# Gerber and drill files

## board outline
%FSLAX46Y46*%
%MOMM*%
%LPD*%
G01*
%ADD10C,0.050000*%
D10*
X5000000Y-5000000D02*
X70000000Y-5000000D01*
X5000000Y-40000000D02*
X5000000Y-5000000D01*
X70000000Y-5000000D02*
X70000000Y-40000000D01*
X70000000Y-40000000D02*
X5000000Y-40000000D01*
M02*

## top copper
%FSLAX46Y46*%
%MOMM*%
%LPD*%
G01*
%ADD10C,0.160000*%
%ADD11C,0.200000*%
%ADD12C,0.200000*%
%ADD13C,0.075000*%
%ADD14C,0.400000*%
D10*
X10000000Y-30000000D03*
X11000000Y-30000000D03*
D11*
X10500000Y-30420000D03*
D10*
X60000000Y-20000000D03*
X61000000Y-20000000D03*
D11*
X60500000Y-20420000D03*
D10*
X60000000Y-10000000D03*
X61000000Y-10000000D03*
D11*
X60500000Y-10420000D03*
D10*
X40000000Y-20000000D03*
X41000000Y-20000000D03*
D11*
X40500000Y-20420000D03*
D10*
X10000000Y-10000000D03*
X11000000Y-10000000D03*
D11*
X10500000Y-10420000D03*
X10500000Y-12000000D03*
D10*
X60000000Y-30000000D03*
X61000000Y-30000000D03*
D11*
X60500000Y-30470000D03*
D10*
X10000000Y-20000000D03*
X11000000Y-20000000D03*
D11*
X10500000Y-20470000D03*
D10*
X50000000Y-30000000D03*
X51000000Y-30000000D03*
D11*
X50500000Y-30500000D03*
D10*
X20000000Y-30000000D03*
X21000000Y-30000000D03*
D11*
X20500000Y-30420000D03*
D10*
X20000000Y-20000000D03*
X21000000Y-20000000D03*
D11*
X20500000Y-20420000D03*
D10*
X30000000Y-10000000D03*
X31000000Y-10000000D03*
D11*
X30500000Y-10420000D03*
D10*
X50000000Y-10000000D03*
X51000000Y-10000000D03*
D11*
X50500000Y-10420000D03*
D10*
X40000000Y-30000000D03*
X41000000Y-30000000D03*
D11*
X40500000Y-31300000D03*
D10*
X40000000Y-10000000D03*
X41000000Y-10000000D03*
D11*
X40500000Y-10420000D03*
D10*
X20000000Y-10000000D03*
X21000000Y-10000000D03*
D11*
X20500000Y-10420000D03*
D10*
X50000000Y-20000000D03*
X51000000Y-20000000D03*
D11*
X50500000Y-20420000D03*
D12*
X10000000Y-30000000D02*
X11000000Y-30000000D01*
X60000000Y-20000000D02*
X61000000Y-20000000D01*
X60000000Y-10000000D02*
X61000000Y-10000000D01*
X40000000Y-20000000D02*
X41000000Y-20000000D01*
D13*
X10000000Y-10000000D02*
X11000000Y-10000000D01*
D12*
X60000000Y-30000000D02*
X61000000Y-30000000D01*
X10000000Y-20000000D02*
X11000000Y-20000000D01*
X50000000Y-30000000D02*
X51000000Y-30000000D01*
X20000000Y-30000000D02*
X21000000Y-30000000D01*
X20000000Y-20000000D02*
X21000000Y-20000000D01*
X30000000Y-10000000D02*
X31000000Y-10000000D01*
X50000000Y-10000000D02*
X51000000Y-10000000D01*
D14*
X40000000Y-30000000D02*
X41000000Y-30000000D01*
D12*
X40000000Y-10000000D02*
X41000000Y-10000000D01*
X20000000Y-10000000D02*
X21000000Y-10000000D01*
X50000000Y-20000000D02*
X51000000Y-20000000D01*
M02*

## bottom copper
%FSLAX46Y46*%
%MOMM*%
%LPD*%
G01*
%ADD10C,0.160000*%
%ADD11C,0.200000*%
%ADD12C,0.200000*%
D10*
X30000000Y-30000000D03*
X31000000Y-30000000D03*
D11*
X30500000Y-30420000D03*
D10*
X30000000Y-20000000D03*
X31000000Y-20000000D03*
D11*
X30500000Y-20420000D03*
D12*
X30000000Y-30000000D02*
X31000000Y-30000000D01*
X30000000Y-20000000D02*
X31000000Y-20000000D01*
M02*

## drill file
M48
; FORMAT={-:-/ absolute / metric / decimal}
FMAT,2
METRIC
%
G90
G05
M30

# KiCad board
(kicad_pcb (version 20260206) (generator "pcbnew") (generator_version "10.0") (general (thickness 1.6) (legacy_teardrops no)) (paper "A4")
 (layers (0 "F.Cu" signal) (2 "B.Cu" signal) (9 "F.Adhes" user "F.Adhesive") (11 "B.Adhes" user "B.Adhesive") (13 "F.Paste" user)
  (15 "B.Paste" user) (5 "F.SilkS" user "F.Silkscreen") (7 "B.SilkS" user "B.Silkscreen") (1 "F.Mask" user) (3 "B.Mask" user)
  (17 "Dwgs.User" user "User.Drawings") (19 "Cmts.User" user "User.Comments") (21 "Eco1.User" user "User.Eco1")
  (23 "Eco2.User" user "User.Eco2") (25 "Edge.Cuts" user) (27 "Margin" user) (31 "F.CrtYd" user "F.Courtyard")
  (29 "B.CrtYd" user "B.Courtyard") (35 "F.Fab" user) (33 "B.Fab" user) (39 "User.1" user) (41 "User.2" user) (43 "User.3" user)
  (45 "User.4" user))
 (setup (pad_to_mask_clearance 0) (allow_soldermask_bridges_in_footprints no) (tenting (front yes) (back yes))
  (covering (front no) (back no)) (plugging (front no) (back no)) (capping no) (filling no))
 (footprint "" (layer "F.Cu") (at 10 30)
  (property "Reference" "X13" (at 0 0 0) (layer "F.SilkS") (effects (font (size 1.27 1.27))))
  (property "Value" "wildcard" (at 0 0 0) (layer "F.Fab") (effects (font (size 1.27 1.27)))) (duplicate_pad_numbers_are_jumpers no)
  (pad "1" smd circle (at 0 0) (size 0.16 0.16) (layers "F.Cu") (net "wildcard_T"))
  (pad "2" smd circle (at 1 0) (size 0.16 0.16) (layers "F.Cu") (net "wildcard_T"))
  (pad "3" smd circle (at 0.5 0.42) (size 0.2 0.2) (layers "F.Cu") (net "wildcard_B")))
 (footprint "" (layer "F.Cu") (at 60 20)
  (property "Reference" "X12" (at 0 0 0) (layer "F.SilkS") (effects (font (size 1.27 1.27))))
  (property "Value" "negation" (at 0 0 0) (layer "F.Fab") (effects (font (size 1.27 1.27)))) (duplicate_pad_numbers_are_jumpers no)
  (pad "1" smd circle (at 0 0) (size 0.16 0.16) (layers "F.Cu") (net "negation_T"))
  (pad "2" smd circle (at 1 0) (size 0.16 0.16) (layers "F.Cu") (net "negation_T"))
  (pad "3" smd circle (at 0.5 0.42) (size 0.2 0.2) (layers "F.Cu") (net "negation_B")))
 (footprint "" (layer "F.Cu") (at 60 10)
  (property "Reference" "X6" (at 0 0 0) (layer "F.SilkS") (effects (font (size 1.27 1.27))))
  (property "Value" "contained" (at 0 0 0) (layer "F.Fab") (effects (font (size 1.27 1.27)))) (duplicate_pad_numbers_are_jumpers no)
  (pad "1" smd circle (at 0 0) (size 0.16 0.16) (layers "F.Cu") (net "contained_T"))
  (pad "2" smd circle (at 1 0) (size 0.16 0.16) (layers "F.Cu") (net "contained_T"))
  (pad "3" smd circle (at 0.5 0.42) (size 0.2 0.2) (layers "F.Cu") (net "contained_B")))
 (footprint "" (layer "F.Cu") (at 40 20)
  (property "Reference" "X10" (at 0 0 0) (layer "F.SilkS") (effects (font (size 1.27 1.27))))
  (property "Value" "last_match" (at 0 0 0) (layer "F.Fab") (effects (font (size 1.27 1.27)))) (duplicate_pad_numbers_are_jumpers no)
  (pad "1" smd circle (at 0 0) (size 0.16 0.16) (layers "F.Cu") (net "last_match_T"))
  (pad "2" smd circle (at 1 0) (size 0.16 0.16) (layers "F.Cu") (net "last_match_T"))
  (pad "3" smd circle (at 0.5 0.42) (size 0.2 0.2) (layers "F.Cu") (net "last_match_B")))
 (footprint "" (layer "F.Cu") (at 10 10)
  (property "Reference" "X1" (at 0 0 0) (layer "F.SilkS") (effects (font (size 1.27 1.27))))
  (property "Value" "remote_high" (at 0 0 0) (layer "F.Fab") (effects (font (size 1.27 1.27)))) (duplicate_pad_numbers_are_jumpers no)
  (pad "1" smd circle (at 0 0) (size 0.16 0.16) (layers "F.Cu") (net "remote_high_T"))
  (pad "2" smd circle (at 1 0) (size 0.16 0.16) (layers "F.Cu") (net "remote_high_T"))
  (pad "3" smd circle (at 0.5 0.42) (size 0.2 0.2) (layers "F.Cu") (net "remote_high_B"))
  (pad "4" smd circle (at 0.5 2) (size 0.2 0.2) (layers "F.Cu") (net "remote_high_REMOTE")))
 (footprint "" (layer "F.Cu") (at 60 30)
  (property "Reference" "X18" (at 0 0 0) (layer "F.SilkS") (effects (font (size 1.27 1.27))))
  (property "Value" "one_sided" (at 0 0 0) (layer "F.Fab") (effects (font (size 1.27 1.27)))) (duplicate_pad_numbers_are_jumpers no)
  (pad "1" smd circle (at 0 0) (size 0.16 0.16) (layers "F.Cu") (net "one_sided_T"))
  (pad "2" smd circle (at 1 0) (size 0.16 0.16) (layers "F.Cu") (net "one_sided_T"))
  (pad "3" smd circle (at 0.5 0.47) (size 0.2 0.2) (layers "F.Cu") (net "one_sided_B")))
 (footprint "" (layer "F.Cu") (at 10 20)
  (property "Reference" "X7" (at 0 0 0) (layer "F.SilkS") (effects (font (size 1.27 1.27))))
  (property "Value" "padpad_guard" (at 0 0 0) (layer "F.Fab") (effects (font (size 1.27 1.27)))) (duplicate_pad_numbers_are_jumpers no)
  (pad "1" smd circle (at 0 0) (size 0.16 0.16) (layers "F.Cu") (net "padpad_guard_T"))
  (pad "2" smd circle (at 1 0) (size 0.16 0.16) (layers "F.Cu") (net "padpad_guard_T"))
  (pad "3" smd circle (at 0.5 0.47) (size 0.2 0.2) (layers "F.Cu") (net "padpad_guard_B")))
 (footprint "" (layer "F.Cu") (at 50 30)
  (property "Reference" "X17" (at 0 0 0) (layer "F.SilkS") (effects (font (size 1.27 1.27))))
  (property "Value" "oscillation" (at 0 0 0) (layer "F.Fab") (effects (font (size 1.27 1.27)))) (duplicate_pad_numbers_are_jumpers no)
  (pad "1" smd circle (at 0 0) (size 0.16 0.16) (layers "F.Cu") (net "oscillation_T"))
  (pad "2" smd circle (at 1 0) (size 0.16 0.16) (layers "F.Cu") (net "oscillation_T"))
  (pad "3" smd circle (at 0.5 0.5) (size 0.2 0.2) (layers "F.Cu") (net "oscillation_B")))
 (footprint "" (layer "F.Cu") (at 20 30)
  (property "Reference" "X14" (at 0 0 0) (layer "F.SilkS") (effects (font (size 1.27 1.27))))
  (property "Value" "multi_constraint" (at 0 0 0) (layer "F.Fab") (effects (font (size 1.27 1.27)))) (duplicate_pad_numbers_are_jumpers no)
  (pad "1" smd circle (at 0 0) (size 0.16 0.16) (layers "F.Cu") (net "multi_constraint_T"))
  (pad "2" smd circle (at 1 0) (size 0.16 0.16) (layers "F.Cu") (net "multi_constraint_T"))
  (pad "3" smd circle (at 0.5 0.42) (size 0.2 0.2) (layers "F.Cu") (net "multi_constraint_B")))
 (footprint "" (layer "F.Cu") (at 30 30)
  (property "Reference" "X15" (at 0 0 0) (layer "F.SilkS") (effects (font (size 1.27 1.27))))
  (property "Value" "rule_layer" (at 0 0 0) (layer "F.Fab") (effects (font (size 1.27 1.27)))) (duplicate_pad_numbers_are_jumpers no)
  (pad "1" smd circle (at 0 0) (size 0.16 0.16) (layers "B.Cu") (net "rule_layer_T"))
  (pad "2" smd circle (at 1 0) (size 0.16 0.16) (layers "B.Cu") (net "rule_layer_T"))
  (pad "3" smd circle (at 0.5 0.42) (size 0.2 0.2) (layers "B.Cu") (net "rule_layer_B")))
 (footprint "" (layer "F.Cu") (at 20 20)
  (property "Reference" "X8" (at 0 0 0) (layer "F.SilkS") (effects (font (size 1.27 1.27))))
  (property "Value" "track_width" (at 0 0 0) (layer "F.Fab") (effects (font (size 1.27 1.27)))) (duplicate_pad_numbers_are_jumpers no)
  (pad "1" smd circle (at 0 0) (size 0.16 0.16) (layers "F.Cu") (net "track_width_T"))
  (pad "2" smd circle (at 1 0) (size 0.16 0.16) (layers "F.Cu") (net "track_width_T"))
  (pad "3" smd circle (at 0.5 0.42) (size 0.2 0.2) (layers "F.Cu") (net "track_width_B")))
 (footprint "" (layer "F.Cu") (at 30 10)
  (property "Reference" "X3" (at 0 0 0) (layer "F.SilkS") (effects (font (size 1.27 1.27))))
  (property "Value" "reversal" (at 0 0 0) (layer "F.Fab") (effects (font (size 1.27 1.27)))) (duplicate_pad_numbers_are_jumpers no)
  (pad "1" smd circle (at 0 0) (size 0.16 0.16) (layers "F.Cu") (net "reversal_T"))
  (pad "2" smd circle (at 1 0) (size 0.16 0.16) (layers "F.Cu") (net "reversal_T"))
  (pad "3" smd circle (at 0.5 0.42) (size 0.2 0.2) (layers "F.Cu") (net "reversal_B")))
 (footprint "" (layer "F.Cu") (at 50 10)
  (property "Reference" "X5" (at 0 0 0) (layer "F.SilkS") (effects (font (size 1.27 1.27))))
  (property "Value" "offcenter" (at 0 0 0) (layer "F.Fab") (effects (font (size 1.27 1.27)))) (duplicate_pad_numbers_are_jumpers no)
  (pad "1" smd circle (at 0 0) (size 0.16 0.16) (layers "F.Cu") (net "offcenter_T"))
  (pad "2" smd circle (at 1 0) (size 0.16 0.16) (layers "F.Cu") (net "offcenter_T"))
  (pad "3" smd circle (at 0.5 0.42) (size 0.2 0.2) (layers "F.Cu") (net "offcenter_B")))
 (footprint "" (layer "F.Cu") (at 40 30)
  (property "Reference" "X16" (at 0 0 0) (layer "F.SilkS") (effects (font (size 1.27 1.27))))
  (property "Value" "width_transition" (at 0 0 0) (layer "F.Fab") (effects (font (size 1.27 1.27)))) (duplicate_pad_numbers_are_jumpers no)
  (pad "1" smd circle (at 0 0) (size 0.16 0.16) (layers "F.Cu") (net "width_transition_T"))
  (pad "2" smd circle (at 1 0) (size 0.16 0.16) (layers "F.Cu") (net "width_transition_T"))
  (pad "3" smd circle (at 0.5 1.3) (size 0.2 0.2) (layers "F.Cu") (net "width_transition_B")))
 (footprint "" (layer "F.Cu") (at 30 20)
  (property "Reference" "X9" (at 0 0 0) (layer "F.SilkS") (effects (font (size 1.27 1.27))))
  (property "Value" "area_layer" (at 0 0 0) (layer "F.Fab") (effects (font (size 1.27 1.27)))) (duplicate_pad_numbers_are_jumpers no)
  (pad "1" smd circle (at 0 0) (size 0.16 0.16) (layers "B.Cu") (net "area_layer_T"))
  (pad "2" smd circle (at 1 0) (size 0.16 0.16) (layers "B.Cu") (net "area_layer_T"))
  (pad "3" smd circle (at 0.5 0.42) (size 0.2 0.2) (layers "B.Cu") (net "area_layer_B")))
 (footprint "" (layer "F.Cu") (at 40 10)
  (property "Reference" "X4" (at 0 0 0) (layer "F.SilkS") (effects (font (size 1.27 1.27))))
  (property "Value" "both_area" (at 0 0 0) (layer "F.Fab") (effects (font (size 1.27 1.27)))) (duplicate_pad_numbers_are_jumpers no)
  (pad "1" smd circle (at 0 0) (size 0.16 0.16) (layers "F.Cu") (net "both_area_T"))
  (pad "2" smd circle (at 1 0) (size 0.16 0.16) (layers "F.Cu") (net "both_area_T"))
  (pad "3" smd circle (at 0.5 0.42) (size 0.2 0.2) (layers "F.Cu") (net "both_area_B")))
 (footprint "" (layer "F.Cu") (at 20 10)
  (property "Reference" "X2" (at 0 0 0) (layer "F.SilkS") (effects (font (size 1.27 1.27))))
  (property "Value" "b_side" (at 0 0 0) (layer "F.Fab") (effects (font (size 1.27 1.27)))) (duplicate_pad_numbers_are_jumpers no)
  (pad "1" smd circle (at 0 0) (size 0.16 0.16) (layers "F.Cu") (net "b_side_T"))
  (pad "2" smd circle (at 1 0) (size 0.16 0.16) (layers "F.Cu") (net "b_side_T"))
  (pad "3" smd circle (at 0.5 0.42) (size 0.2 0.2) (layers "F.Cu") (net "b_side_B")))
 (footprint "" (layer "F.Cu") (at 50 20)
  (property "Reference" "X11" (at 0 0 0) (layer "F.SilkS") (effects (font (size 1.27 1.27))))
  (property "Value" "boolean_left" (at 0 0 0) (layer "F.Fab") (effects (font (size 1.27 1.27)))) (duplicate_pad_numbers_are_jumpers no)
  (pad "1" smd circle (at 0 0) (size 0.16 0.16) (layers "F.Cu") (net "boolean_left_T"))
  (pad "2" smd circle (at 1 0) (size 0.16 0.16) (layers "F.Cu") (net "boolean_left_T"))
  (pad "3" smd circle (at 0.5 0.42) (size 0.2 0.2) (layers "F.Cu") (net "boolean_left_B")))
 (gr_line (start 5 5) (end 70 5) (stroke (width 0.05) (type default)) (layer "Edge.Cuts"))
 (gr_line (start 5 40) (end 5 5) (stroke (width 0.05) (type default)) (layer "Edge.Cuts"))
 (gr_line (start 70 5) (end 70 40) (stroke (width 0.05) (type default)) (layer "Edge.Cuts"))
 (gr_line (start 70 40) (end 5 40) (stroke (width 0.05) (type default)) (layer "Edge.Cuts"))
 (segment (start 10 30) (end 11 30) (width 0.2) (layer "F.Cu") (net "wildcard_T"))
 (segment (start 60 20) (end 61 20) (width 0.2) (layer "F.Cu") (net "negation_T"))
 (segment (start 60 10) (end 61 10) (width 0.2) (layer "F.Cu") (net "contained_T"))
 (segment (start 40 20) (end 41 20) (width 0.2) (layer "F.Cu") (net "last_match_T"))
 (segment (start 10 10) (end 11 10) (width 0.075) (layer "F.Cu") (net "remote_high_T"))
 (segment (start 60 30) (end 61 30) (width 0.2) (layer "F.Cu") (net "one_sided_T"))
 (segment (start 10 20) (end 11 20) (width 0.2) (layer "F.Cu") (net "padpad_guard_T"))
 (segment (start 50 30) (end 51 30) (width 0.2) (layer "F.Cu") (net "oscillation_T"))
 (segment (start 20 30) (end 21 30) (width 0.2) (layer "F.Cu") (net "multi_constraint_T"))
 (segment (start 30 30) (end 31 30) (width 0.2) (layer "B.Cu") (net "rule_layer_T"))
 (segment (start 20 20) (end 21 20) (width 0.2) (layer "F.Cu") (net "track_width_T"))
 (segment (start 30 10) (end 31 10) (width 0.2) (layer "F.Cu") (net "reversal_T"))
 (segment (start 50 10) (end 51 10) (width 0.2) (layer "F.Cu") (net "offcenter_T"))
 (segment (start 40 30) (end 41 30) (width 0.4) (layer "F.Cu") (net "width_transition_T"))
 (segment (start 30 20) (end 31 20) (width 0.2) (layer "B.Cu") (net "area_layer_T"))
 (segment (start 40 10) (end 41 10) (width 0.2) (layer "F.Cu") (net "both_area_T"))
 (segment (start 20 10) (end 21 10) (width 0.2) (layer "F.Cu") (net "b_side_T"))
 (segment (start 50 20) (end 51 20) (width 0.2) (layer "F.Cu") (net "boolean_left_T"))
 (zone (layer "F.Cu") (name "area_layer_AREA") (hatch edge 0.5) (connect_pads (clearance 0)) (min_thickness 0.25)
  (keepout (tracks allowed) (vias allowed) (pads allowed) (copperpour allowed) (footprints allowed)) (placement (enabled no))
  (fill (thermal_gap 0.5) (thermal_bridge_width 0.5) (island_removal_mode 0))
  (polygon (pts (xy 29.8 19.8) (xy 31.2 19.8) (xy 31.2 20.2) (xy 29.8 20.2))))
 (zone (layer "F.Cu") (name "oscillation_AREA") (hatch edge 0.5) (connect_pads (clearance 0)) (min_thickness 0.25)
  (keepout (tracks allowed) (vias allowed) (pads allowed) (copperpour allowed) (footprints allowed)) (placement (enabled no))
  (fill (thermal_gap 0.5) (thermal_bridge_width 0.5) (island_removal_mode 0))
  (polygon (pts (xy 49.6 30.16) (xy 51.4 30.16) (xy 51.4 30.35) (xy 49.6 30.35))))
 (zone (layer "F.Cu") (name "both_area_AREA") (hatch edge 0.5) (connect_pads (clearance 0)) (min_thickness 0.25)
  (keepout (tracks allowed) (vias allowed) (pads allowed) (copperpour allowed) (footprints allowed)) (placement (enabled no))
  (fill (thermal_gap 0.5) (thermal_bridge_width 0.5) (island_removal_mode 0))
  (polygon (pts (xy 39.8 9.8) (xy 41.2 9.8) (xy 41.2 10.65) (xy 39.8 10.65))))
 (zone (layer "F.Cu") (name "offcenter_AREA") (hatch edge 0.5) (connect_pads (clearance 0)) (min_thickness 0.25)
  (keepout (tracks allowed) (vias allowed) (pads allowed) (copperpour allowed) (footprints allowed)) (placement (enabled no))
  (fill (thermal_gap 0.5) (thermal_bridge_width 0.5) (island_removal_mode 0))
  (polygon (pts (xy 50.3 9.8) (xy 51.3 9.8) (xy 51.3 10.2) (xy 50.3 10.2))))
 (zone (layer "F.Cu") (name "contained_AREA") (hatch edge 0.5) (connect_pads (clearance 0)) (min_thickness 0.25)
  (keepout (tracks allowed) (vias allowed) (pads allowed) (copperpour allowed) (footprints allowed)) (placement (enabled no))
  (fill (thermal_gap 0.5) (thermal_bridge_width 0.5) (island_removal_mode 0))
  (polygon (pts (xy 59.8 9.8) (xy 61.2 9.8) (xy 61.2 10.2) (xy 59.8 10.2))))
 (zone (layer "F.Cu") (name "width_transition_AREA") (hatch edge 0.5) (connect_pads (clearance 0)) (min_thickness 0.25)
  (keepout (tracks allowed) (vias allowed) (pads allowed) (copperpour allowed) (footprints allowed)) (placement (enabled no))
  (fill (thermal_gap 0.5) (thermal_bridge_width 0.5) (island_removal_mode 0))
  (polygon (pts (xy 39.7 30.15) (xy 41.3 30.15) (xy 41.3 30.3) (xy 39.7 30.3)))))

